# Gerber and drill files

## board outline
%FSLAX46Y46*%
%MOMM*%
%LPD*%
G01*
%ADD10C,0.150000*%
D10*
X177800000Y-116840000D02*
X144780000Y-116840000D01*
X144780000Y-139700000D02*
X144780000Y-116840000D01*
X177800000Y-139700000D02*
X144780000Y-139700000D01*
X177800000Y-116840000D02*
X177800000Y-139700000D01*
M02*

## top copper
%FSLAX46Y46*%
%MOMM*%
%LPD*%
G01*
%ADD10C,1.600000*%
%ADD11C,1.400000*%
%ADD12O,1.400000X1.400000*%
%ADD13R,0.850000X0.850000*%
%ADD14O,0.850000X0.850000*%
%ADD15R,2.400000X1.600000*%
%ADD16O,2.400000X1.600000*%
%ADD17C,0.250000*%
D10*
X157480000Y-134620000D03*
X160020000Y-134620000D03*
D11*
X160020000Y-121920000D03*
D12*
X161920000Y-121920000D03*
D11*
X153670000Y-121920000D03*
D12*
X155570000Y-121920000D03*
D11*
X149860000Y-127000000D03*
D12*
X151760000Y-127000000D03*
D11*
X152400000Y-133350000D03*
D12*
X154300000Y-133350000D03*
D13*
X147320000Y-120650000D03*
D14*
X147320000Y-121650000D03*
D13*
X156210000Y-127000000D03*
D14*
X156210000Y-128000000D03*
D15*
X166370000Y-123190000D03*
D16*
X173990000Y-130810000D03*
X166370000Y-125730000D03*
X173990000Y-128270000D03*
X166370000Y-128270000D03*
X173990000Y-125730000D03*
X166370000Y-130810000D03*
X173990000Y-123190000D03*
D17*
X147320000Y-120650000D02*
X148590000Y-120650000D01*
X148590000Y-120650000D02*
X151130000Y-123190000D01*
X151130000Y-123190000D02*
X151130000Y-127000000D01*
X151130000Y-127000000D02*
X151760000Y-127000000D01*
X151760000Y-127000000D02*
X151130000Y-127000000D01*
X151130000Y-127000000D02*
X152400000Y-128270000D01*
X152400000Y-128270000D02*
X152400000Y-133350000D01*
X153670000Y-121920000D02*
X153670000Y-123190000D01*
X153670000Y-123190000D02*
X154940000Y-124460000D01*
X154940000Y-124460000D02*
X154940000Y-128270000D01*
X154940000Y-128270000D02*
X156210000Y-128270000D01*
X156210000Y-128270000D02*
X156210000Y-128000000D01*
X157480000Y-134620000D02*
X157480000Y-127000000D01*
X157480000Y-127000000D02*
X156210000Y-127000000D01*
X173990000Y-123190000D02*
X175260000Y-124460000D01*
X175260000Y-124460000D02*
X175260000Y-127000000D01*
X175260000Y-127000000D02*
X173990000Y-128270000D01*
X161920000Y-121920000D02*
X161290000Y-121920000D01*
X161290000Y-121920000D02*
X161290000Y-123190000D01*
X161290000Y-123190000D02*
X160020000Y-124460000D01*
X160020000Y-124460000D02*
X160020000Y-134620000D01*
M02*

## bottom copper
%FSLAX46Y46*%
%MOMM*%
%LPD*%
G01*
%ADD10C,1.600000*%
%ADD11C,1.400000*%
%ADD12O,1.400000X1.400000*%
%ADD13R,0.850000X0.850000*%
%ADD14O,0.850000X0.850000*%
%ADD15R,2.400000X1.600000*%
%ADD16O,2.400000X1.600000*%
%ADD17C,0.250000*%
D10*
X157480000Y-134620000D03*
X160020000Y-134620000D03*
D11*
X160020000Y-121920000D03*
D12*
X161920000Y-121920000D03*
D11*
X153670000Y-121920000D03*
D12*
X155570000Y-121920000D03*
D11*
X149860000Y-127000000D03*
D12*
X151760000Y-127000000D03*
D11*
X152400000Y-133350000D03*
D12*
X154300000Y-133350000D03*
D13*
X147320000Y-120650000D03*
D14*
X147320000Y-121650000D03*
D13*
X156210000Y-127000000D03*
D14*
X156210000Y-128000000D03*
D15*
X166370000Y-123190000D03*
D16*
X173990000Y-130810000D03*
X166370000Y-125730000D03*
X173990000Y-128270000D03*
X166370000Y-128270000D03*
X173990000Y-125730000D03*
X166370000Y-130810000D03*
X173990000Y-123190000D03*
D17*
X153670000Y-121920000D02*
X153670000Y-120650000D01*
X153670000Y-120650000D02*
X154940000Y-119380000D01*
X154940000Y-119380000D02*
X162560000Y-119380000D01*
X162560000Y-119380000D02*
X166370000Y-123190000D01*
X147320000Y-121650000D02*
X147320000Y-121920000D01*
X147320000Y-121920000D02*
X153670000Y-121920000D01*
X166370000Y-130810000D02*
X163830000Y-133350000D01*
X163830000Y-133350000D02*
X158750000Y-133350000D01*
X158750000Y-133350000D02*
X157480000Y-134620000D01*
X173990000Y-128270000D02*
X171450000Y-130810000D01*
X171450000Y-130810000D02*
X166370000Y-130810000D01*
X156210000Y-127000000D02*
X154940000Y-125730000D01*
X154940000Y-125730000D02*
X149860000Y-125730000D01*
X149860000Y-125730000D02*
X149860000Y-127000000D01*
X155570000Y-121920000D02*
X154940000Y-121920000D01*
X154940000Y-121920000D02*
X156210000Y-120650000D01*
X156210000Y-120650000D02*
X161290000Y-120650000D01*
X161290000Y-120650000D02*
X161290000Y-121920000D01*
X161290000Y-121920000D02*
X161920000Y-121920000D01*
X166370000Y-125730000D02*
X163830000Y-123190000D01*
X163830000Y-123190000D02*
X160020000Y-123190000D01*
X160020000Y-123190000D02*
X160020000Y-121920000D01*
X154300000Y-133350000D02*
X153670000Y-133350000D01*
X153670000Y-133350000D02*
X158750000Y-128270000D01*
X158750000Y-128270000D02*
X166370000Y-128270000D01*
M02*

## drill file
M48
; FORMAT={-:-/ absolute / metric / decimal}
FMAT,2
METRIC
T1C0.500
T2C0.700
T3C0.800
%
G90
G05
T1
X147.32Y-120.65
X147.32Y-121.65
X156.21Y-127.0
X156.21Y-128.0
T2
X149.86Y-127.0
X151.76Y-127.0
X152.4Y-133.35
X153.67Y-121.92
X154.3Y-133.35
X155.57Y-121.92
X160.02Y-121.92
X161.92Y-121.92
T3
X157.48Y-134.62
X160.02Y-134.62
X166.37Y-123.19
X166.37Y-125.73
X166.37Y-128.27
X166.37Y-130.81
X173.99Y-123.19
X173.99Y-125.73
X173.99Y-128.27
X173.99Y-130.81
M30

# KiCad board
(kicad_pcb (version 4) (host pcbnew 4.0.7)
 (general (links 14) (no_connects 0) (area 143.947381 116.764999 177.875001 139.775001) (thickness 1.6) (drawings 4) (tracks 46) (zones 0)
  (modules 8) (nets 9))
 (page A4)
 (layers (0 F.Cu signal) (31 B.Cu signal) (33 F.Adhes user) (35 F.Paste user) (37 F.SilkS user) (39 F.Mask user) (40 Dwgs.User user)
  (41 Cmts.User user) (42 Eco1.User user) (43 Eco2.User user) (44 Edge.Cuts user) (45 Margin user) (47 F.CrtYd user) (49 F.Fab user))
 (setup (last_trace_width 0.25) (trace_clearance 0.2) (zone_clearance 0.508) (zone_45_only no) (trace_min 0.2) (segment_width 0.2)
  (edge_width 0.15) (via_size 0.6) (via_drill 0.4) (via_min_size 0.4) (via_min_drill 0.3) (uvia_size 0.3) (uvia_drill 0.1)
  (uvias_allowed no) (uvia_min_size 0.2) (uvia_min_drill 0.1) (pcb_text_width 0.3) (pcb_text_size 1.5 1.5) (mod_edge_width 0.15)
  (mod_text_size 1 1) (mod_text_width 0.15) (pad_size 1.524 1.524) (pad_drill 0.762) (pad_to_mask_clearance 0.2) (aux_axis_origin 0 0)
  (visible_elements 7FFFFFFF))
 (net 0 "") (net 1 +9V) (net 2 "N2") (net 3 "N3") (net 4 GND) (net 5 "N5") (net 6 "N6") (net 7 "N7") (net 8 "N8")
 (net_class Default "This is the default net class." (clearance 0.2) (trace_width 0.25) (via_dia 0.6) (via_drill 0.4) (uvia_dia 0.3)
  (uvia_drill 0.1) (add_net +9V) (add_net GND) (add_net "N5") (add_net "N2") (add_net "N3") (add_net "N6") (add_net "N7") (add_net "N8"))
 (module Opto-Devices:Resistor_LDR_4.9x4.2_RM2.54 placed (layer F.Cu) (at 157.48 134.62)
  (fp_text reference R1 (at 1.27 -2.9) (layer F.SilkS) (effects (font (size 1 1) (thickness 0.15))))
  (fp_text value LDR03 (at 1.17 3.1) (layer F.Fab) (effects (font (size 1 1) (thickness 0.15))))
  (pad 1 thru_hole circle (at 0 0) (size 1.6 1.6) (drill 0.8) (layers *.Cu *.Mask) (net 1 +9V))
  (pad 2 thru_hole circle (at 2.54 0) (size 1.6 1.6) (drill 0.8) (layers *.Cu *.Mask) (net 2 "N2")))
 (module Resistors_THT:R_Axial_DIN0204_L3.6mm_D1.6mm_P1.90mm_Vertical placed (layer F.Cu) (at 160.02 121.92)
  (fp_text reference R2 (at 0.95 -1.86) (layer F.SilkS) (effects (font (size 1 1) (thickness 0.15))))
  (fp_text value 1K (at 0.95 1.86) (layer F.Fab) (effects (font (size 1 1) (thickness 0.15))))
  (pad 1 thru_hole circle (at 0 0) (size 1.4 1.4) (drill 0.7) (layers *.Cu *.Mask) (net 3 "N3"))
  (pad 2 thru_hole oval (at 1.9 0) (size 1.4 1.4) (drill 0.7) (layers *.Cu *.Mask) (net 2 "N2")))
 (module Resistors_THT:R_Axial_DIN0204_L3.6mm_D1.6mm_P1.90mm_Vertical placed (layer F.Cu) (at 153.67 121.92)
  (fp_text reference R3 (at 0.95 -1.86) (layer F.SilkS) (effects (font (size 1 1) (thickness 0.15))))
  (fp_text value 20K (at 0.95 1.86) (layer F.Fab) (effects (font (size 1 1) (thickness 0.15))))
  (pad 1 thru_hole circle (at 0 0) (size 1.4 1.4) (drill 0.7) (layers *.Cu *.Mask) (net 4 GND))
  (pad 2 thru_hole oval (at 1.9 0) (size 1.4 1.4) (drill 0.7) (layers *.Cu *.Mask) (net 2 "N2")))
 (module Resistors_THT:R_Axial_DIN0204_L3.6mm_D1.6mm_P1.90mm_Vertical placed (layer F.Cu) (at 149.86 127)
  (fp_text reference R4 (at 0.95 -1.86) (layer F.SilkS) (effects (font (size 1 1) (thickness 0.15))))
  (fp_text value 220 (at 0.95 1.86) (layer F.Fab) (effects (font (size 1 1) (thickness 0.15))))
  (pad 1 thru_hole circle (at 0 0) (size 1.4 1.4) (drill 0.7) (layers *.Cu *.Mask) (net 1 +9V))
  (pad 2 thru_hole oval (at 1.9 0) (size 1.4 1.4) (drill 0.7) (layers *.Cu *.Mask) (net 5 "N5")))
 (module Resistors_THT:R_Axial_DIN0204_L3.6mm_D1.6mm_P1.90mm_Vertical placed (layer F.Cu) (at 152.4 133.35)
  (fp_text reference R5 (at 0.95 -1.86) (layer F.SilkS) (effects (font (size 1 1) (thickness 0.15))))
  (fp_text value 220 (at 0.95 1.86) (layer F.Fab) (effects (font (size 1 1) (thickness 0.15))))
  (pad 1 thru_hole circle (at 0 0) (size 1.4 1.4) (drill 0.7) (layers *.Cu *.Mask) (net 5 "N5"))
  (pad 2 thru_hole oval (at 1.9 0) (size 1.4 1.4) (drill 0.7) (layers *.Cu *.Mask) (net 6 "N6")))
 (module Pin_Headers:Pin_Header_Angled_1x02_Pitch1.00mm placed (layer F.Cu) (at 147.32 120.65)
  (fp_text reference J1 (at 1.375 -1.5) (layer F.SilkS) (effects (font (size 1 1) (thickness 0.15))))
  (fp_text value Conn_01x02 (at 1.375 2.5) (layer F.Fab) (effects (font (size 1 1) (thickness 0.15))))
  (pad 1 thru_hole rect (at 0 0) (size 0.85 0.85) (drill 0.5) (layers *.Cu *.Mask) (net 5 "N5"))
  (pad 2 thru_hole oval (at 0 1) (size 0.85 0.85) (drill 0.5) (layers *.Cu *.Mask) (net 4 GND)))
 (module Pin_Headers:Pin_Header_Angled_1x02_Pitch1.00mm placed (layer F.Cu) (at 156.21 127)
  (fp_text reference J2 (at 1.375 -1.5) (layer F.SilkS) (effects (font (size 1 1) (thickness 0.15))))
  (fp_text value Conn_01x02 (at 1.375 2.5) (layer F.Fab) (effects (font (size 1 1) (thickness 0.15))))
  (pad 1 thru_hole rect (at 0 0) (size 0.85 0.85) (drill 0.5) (layers *.Cu *.Mask) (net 1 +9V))
  (pad 2 thru_hole oval (at 0 1) (size 0.85 0.85) (drill 0.5) (layers *.Cu *.Mask) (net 4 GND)))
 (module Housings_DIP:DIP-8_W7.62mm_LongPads (layer F.Cu) (at 166.37 123.19)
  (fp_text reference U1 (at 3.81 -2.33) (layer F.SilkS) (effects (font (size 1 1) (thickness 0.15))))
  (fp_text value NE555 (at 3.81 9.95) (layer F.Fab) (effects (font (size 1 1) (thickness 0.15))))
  (pad 1 thru_hole rect (at 0 0) (size 2.4 1.6) (drill 0.8) (layers *.Cu *.Mask) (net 4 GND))
  (pad 5 thru_hole oval (at 7.62 7.62) (size 2.4 1.6) (drill 0.8) (layers *.Cu *.Mask) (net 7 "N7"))
  (pad 2 thru_hole oval (at 0 2.54) (size 2.4 1.6) (drill 0.8) (layers *.Cu *.Mask) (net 3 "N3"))
  (pad 6 thru_hole oval (at 7.62 5.08) (size 2.4 1.6) (drill 0.8) (layers *.Cu *.Mask) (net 1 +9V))
  (pad 3 thru_hole oval (at 0 5.08) (size 2.4 1.6) (drill 0.8) (layers *.Cu *.Mask) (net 6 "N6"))
  (pad 7 thru_hole oval (at 7.62 2.54) (size 2.4 1.6) (drill 0.8) (layers *.Cu *.Mask) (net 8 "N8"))
  (pad 4 thru_hole oval (at 0 7.62) (size 2.4 1.6) (drill 0.8) (layers *.Cu *.Mask) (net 1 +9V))
  (pad 8 thru_hole oval (at 7.62 0) (size 2.4 1.6) (drill 0.8) (layers *.Cu *.Mask) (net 1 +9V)))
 (gr_line (start 177.8 116.84) (end 144.78 116.84) (angle 90) (layer Edge.Cuts) (width 0.15))
 (gr_line (start 144.78 139.7) (end 144.78 116.84) (angle 90) (layer Edge.Cuts) (width 0.15))
 (gr_line (start 177.8 139.7) (end 144.78 139.7) (angle 90) (layer Edge.Cuts) (width 0.15))
 (gr_line (start 177.8 116.84) (end 177.8 139.7) (angle 90) (layer Edge.Cuts) (width 0.15))
 (segment (start 147.32 120.65) (end 148.59 120.65) (width 0.25) (layer F.Cu) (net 5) (status 80000))
 (segment (start 148.59 120.65) (end 151.13 123.19) (width 0.25) (layer F.Cu) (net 5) (status 80000))
 (segment (start 151.13 123.19) (end 151.13 127) (width 0.25) (layer F.Cu) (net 5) (status 80000))
 (segment (start 151.13 127) (end 151.76 127) (width 0.25) (layer F.Cu) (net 5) (status 80000))
 (segment (start 151.76 127) (end 151.13 127) (width 0.25) (layer F.Cu) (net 5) (status 80000))
 (segment (start 151.13 127) (end 152.4 128.27) (width 0.25) (layer F.Cu) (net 5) (status 80000))
 (segment (start 152.4 128.27) (end 152.4 133.35) (width 0.25) (layer F.Cu) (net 5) (status 80000))
 (segment (start 153.67 121.92) (end 153.67 120.65) (width 0.25) (layer B.Cu) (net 4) (status 80000))
 (segment (start 153.67 120.65) (end 154.94 119.38) (width 0.25) (layer B.Cu) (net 4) (status 80000))
 (segment (start 154.94 119.38) (end 162.56 119.38) (width 0.25) (layer B.Cu) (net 4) (status 80000))
 (segment (start 162.56 119.38) (end 166.37 123.19) (width 0.25) (layer B.Cu) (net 4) (status 80000))
 (segment (start 153.67 121.92) (end 153.67 123.19) (width 0.25) (layer F.Cu) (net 4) (status 80000))
 (segment (start 153.67 123.19) (end 154.94 124.46) (width 0.25) (layer F.Cu) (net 4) (status 80000))
 (segment (start 154.94 124.46) (end 154.94 128.27) (width 0.25) (layer F.Cu) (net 4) (status 80000))
 (segment (start 154.94 128.27) (end 156.21 128.27) (width 0.25) (layer F.Cu) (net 4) (status 80000))
 (segment (start 156.21 128.27) (end 156.21 128) (width 0.25) (layer F.Cu) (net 4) (status 80000))
 (segment (start 147.32 121.65) (end 147.32 121.92) (width 0.25) (layer B.Cu) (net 4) (status 80000))
 (segment (start 147.32 121.92) (end 153.67 121.92) (width 0.25) (layer B.Cu) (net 4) (status 80000))
 (segment (start 166.37 130.81) (end 163.83 133.35) (width 0.25) (layer B.Cu) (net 1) (status 80000))
 (segment (start 163.83 133.35) (end 158.75 133.35) (width 0.25) (layer B.Cu) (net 1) (status 80000))
 (segment (start 158.75 133.35) (end 157.48 134.62) (width 0.25) (layer B.Cu) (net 1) (status 80000))
 (segment (start 173.99 128.27) (end 171.45 130.81) (width 0.25) (layer B.Cu) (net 1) (status 80000))
 (segment (start 171.45 130.81) (end 166.37 130.81) (width 0.25) (layer B.Cu) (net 1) (status 80000))
 (segment (start 157.48 134.62) (end 157.48 127) (width 0.25) (layer F.Cu) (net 1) (status 80000))
 (segment (start 157.48 127) (end 156.21 127) (width 0.25) (layer F.Cu) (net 1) (status 80000))
 (segment (start 156.21 127) (end 154.94 125.73) (width 0.25) (layer B.Cu) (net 1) (status 80000))
 (segment (start 154.94 125.73) (end 149.86 125.73) (width 0.25) (layer B.Cu) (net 1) (status 80000))
 (segment (start 149.86 125.73) (end 149.86 127) (width 0.25) (layer B.Cu) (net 1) (status 80000))
 (segment (start 173.99 123.19) (end 175.26 124.46) (width 0.25) (layer F.Cu) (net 1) (status 80000))
 (segment (start 175.26 124.46) (end 175.26 127) (width 0.25) (layer F.Cu) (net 1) (status 80000))
 (segment (start 175.26 127) (end 173.99 128.27) (width 0.25) (layer F.Cu) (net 1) (status 80000))
 (segment (start 161.92 121.92) (end 161.29 121.92) (width 0.25) (layer F.Cu) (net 2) (status 80000))
 (segment (start 161.29 121.92) (end 161.29 123.19) (width 0.25) (layer F.Cu) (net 2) (status 80000))
 (segment (start 161.29 123.19) (end 160.02 124.46) (width 0.25) (layer F.Cu) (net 2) (status 80000))
 (segment (start 160.02 124.46) (end 160.02 134.62) (width 0.25) (layer F.Cu) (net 2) (status 80000))
 (segment (start 155.57 121.92) (end 154.94 121.92) (width 0.25) (layer B.Cu) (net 2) (status 80000))
 (segment (start 154.94 121.92) (end 156.21 120.65) (width 0.25) (layer B.Cu) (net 2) (status 80000))
 (segment (start 156.21 120.65) (end 161.29 120.65) (width 0.25) (layer B.Cu) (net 2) (status 80000))
 (segment (start 161.29 120.65) (end 161.29 121.92) (width 0.25) (layer B.Cu) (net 2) (status 80000))
 (segment (start 161.29 121.92) (end 161.92 121.92) (width 0.25) (layer B.Cu) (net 2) (status 80000))
 (segment (start 166.37 125.73) (end 163.83 123.19) (width 0.25) (layer B.Cu) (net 3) (status 80000))
 (segment (start 163.83 123.19) (end 160.02 123.19) (width 0.25) (layer B.Cu) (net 3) (status 80000))
 (segment (start 160.02 123.19) (end 160.02 121.92) (width 0.25) (layer B.Cu) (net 3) (status 80000))
 (segment (start 154.3 133.35) (end 153.67 133.35) (width 0.25) (layer B.Cu) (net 6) (status 80000))
 (segment (start 153.67 133.35) (end 158.75 128.27) (width 0.25) (layer B.Cu) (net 6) (status 80000))
 (segment (start 158.75 128.27) (end 166.37 128.27) (width 0.25) (layer B.Cu) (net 6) (status 80000)))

